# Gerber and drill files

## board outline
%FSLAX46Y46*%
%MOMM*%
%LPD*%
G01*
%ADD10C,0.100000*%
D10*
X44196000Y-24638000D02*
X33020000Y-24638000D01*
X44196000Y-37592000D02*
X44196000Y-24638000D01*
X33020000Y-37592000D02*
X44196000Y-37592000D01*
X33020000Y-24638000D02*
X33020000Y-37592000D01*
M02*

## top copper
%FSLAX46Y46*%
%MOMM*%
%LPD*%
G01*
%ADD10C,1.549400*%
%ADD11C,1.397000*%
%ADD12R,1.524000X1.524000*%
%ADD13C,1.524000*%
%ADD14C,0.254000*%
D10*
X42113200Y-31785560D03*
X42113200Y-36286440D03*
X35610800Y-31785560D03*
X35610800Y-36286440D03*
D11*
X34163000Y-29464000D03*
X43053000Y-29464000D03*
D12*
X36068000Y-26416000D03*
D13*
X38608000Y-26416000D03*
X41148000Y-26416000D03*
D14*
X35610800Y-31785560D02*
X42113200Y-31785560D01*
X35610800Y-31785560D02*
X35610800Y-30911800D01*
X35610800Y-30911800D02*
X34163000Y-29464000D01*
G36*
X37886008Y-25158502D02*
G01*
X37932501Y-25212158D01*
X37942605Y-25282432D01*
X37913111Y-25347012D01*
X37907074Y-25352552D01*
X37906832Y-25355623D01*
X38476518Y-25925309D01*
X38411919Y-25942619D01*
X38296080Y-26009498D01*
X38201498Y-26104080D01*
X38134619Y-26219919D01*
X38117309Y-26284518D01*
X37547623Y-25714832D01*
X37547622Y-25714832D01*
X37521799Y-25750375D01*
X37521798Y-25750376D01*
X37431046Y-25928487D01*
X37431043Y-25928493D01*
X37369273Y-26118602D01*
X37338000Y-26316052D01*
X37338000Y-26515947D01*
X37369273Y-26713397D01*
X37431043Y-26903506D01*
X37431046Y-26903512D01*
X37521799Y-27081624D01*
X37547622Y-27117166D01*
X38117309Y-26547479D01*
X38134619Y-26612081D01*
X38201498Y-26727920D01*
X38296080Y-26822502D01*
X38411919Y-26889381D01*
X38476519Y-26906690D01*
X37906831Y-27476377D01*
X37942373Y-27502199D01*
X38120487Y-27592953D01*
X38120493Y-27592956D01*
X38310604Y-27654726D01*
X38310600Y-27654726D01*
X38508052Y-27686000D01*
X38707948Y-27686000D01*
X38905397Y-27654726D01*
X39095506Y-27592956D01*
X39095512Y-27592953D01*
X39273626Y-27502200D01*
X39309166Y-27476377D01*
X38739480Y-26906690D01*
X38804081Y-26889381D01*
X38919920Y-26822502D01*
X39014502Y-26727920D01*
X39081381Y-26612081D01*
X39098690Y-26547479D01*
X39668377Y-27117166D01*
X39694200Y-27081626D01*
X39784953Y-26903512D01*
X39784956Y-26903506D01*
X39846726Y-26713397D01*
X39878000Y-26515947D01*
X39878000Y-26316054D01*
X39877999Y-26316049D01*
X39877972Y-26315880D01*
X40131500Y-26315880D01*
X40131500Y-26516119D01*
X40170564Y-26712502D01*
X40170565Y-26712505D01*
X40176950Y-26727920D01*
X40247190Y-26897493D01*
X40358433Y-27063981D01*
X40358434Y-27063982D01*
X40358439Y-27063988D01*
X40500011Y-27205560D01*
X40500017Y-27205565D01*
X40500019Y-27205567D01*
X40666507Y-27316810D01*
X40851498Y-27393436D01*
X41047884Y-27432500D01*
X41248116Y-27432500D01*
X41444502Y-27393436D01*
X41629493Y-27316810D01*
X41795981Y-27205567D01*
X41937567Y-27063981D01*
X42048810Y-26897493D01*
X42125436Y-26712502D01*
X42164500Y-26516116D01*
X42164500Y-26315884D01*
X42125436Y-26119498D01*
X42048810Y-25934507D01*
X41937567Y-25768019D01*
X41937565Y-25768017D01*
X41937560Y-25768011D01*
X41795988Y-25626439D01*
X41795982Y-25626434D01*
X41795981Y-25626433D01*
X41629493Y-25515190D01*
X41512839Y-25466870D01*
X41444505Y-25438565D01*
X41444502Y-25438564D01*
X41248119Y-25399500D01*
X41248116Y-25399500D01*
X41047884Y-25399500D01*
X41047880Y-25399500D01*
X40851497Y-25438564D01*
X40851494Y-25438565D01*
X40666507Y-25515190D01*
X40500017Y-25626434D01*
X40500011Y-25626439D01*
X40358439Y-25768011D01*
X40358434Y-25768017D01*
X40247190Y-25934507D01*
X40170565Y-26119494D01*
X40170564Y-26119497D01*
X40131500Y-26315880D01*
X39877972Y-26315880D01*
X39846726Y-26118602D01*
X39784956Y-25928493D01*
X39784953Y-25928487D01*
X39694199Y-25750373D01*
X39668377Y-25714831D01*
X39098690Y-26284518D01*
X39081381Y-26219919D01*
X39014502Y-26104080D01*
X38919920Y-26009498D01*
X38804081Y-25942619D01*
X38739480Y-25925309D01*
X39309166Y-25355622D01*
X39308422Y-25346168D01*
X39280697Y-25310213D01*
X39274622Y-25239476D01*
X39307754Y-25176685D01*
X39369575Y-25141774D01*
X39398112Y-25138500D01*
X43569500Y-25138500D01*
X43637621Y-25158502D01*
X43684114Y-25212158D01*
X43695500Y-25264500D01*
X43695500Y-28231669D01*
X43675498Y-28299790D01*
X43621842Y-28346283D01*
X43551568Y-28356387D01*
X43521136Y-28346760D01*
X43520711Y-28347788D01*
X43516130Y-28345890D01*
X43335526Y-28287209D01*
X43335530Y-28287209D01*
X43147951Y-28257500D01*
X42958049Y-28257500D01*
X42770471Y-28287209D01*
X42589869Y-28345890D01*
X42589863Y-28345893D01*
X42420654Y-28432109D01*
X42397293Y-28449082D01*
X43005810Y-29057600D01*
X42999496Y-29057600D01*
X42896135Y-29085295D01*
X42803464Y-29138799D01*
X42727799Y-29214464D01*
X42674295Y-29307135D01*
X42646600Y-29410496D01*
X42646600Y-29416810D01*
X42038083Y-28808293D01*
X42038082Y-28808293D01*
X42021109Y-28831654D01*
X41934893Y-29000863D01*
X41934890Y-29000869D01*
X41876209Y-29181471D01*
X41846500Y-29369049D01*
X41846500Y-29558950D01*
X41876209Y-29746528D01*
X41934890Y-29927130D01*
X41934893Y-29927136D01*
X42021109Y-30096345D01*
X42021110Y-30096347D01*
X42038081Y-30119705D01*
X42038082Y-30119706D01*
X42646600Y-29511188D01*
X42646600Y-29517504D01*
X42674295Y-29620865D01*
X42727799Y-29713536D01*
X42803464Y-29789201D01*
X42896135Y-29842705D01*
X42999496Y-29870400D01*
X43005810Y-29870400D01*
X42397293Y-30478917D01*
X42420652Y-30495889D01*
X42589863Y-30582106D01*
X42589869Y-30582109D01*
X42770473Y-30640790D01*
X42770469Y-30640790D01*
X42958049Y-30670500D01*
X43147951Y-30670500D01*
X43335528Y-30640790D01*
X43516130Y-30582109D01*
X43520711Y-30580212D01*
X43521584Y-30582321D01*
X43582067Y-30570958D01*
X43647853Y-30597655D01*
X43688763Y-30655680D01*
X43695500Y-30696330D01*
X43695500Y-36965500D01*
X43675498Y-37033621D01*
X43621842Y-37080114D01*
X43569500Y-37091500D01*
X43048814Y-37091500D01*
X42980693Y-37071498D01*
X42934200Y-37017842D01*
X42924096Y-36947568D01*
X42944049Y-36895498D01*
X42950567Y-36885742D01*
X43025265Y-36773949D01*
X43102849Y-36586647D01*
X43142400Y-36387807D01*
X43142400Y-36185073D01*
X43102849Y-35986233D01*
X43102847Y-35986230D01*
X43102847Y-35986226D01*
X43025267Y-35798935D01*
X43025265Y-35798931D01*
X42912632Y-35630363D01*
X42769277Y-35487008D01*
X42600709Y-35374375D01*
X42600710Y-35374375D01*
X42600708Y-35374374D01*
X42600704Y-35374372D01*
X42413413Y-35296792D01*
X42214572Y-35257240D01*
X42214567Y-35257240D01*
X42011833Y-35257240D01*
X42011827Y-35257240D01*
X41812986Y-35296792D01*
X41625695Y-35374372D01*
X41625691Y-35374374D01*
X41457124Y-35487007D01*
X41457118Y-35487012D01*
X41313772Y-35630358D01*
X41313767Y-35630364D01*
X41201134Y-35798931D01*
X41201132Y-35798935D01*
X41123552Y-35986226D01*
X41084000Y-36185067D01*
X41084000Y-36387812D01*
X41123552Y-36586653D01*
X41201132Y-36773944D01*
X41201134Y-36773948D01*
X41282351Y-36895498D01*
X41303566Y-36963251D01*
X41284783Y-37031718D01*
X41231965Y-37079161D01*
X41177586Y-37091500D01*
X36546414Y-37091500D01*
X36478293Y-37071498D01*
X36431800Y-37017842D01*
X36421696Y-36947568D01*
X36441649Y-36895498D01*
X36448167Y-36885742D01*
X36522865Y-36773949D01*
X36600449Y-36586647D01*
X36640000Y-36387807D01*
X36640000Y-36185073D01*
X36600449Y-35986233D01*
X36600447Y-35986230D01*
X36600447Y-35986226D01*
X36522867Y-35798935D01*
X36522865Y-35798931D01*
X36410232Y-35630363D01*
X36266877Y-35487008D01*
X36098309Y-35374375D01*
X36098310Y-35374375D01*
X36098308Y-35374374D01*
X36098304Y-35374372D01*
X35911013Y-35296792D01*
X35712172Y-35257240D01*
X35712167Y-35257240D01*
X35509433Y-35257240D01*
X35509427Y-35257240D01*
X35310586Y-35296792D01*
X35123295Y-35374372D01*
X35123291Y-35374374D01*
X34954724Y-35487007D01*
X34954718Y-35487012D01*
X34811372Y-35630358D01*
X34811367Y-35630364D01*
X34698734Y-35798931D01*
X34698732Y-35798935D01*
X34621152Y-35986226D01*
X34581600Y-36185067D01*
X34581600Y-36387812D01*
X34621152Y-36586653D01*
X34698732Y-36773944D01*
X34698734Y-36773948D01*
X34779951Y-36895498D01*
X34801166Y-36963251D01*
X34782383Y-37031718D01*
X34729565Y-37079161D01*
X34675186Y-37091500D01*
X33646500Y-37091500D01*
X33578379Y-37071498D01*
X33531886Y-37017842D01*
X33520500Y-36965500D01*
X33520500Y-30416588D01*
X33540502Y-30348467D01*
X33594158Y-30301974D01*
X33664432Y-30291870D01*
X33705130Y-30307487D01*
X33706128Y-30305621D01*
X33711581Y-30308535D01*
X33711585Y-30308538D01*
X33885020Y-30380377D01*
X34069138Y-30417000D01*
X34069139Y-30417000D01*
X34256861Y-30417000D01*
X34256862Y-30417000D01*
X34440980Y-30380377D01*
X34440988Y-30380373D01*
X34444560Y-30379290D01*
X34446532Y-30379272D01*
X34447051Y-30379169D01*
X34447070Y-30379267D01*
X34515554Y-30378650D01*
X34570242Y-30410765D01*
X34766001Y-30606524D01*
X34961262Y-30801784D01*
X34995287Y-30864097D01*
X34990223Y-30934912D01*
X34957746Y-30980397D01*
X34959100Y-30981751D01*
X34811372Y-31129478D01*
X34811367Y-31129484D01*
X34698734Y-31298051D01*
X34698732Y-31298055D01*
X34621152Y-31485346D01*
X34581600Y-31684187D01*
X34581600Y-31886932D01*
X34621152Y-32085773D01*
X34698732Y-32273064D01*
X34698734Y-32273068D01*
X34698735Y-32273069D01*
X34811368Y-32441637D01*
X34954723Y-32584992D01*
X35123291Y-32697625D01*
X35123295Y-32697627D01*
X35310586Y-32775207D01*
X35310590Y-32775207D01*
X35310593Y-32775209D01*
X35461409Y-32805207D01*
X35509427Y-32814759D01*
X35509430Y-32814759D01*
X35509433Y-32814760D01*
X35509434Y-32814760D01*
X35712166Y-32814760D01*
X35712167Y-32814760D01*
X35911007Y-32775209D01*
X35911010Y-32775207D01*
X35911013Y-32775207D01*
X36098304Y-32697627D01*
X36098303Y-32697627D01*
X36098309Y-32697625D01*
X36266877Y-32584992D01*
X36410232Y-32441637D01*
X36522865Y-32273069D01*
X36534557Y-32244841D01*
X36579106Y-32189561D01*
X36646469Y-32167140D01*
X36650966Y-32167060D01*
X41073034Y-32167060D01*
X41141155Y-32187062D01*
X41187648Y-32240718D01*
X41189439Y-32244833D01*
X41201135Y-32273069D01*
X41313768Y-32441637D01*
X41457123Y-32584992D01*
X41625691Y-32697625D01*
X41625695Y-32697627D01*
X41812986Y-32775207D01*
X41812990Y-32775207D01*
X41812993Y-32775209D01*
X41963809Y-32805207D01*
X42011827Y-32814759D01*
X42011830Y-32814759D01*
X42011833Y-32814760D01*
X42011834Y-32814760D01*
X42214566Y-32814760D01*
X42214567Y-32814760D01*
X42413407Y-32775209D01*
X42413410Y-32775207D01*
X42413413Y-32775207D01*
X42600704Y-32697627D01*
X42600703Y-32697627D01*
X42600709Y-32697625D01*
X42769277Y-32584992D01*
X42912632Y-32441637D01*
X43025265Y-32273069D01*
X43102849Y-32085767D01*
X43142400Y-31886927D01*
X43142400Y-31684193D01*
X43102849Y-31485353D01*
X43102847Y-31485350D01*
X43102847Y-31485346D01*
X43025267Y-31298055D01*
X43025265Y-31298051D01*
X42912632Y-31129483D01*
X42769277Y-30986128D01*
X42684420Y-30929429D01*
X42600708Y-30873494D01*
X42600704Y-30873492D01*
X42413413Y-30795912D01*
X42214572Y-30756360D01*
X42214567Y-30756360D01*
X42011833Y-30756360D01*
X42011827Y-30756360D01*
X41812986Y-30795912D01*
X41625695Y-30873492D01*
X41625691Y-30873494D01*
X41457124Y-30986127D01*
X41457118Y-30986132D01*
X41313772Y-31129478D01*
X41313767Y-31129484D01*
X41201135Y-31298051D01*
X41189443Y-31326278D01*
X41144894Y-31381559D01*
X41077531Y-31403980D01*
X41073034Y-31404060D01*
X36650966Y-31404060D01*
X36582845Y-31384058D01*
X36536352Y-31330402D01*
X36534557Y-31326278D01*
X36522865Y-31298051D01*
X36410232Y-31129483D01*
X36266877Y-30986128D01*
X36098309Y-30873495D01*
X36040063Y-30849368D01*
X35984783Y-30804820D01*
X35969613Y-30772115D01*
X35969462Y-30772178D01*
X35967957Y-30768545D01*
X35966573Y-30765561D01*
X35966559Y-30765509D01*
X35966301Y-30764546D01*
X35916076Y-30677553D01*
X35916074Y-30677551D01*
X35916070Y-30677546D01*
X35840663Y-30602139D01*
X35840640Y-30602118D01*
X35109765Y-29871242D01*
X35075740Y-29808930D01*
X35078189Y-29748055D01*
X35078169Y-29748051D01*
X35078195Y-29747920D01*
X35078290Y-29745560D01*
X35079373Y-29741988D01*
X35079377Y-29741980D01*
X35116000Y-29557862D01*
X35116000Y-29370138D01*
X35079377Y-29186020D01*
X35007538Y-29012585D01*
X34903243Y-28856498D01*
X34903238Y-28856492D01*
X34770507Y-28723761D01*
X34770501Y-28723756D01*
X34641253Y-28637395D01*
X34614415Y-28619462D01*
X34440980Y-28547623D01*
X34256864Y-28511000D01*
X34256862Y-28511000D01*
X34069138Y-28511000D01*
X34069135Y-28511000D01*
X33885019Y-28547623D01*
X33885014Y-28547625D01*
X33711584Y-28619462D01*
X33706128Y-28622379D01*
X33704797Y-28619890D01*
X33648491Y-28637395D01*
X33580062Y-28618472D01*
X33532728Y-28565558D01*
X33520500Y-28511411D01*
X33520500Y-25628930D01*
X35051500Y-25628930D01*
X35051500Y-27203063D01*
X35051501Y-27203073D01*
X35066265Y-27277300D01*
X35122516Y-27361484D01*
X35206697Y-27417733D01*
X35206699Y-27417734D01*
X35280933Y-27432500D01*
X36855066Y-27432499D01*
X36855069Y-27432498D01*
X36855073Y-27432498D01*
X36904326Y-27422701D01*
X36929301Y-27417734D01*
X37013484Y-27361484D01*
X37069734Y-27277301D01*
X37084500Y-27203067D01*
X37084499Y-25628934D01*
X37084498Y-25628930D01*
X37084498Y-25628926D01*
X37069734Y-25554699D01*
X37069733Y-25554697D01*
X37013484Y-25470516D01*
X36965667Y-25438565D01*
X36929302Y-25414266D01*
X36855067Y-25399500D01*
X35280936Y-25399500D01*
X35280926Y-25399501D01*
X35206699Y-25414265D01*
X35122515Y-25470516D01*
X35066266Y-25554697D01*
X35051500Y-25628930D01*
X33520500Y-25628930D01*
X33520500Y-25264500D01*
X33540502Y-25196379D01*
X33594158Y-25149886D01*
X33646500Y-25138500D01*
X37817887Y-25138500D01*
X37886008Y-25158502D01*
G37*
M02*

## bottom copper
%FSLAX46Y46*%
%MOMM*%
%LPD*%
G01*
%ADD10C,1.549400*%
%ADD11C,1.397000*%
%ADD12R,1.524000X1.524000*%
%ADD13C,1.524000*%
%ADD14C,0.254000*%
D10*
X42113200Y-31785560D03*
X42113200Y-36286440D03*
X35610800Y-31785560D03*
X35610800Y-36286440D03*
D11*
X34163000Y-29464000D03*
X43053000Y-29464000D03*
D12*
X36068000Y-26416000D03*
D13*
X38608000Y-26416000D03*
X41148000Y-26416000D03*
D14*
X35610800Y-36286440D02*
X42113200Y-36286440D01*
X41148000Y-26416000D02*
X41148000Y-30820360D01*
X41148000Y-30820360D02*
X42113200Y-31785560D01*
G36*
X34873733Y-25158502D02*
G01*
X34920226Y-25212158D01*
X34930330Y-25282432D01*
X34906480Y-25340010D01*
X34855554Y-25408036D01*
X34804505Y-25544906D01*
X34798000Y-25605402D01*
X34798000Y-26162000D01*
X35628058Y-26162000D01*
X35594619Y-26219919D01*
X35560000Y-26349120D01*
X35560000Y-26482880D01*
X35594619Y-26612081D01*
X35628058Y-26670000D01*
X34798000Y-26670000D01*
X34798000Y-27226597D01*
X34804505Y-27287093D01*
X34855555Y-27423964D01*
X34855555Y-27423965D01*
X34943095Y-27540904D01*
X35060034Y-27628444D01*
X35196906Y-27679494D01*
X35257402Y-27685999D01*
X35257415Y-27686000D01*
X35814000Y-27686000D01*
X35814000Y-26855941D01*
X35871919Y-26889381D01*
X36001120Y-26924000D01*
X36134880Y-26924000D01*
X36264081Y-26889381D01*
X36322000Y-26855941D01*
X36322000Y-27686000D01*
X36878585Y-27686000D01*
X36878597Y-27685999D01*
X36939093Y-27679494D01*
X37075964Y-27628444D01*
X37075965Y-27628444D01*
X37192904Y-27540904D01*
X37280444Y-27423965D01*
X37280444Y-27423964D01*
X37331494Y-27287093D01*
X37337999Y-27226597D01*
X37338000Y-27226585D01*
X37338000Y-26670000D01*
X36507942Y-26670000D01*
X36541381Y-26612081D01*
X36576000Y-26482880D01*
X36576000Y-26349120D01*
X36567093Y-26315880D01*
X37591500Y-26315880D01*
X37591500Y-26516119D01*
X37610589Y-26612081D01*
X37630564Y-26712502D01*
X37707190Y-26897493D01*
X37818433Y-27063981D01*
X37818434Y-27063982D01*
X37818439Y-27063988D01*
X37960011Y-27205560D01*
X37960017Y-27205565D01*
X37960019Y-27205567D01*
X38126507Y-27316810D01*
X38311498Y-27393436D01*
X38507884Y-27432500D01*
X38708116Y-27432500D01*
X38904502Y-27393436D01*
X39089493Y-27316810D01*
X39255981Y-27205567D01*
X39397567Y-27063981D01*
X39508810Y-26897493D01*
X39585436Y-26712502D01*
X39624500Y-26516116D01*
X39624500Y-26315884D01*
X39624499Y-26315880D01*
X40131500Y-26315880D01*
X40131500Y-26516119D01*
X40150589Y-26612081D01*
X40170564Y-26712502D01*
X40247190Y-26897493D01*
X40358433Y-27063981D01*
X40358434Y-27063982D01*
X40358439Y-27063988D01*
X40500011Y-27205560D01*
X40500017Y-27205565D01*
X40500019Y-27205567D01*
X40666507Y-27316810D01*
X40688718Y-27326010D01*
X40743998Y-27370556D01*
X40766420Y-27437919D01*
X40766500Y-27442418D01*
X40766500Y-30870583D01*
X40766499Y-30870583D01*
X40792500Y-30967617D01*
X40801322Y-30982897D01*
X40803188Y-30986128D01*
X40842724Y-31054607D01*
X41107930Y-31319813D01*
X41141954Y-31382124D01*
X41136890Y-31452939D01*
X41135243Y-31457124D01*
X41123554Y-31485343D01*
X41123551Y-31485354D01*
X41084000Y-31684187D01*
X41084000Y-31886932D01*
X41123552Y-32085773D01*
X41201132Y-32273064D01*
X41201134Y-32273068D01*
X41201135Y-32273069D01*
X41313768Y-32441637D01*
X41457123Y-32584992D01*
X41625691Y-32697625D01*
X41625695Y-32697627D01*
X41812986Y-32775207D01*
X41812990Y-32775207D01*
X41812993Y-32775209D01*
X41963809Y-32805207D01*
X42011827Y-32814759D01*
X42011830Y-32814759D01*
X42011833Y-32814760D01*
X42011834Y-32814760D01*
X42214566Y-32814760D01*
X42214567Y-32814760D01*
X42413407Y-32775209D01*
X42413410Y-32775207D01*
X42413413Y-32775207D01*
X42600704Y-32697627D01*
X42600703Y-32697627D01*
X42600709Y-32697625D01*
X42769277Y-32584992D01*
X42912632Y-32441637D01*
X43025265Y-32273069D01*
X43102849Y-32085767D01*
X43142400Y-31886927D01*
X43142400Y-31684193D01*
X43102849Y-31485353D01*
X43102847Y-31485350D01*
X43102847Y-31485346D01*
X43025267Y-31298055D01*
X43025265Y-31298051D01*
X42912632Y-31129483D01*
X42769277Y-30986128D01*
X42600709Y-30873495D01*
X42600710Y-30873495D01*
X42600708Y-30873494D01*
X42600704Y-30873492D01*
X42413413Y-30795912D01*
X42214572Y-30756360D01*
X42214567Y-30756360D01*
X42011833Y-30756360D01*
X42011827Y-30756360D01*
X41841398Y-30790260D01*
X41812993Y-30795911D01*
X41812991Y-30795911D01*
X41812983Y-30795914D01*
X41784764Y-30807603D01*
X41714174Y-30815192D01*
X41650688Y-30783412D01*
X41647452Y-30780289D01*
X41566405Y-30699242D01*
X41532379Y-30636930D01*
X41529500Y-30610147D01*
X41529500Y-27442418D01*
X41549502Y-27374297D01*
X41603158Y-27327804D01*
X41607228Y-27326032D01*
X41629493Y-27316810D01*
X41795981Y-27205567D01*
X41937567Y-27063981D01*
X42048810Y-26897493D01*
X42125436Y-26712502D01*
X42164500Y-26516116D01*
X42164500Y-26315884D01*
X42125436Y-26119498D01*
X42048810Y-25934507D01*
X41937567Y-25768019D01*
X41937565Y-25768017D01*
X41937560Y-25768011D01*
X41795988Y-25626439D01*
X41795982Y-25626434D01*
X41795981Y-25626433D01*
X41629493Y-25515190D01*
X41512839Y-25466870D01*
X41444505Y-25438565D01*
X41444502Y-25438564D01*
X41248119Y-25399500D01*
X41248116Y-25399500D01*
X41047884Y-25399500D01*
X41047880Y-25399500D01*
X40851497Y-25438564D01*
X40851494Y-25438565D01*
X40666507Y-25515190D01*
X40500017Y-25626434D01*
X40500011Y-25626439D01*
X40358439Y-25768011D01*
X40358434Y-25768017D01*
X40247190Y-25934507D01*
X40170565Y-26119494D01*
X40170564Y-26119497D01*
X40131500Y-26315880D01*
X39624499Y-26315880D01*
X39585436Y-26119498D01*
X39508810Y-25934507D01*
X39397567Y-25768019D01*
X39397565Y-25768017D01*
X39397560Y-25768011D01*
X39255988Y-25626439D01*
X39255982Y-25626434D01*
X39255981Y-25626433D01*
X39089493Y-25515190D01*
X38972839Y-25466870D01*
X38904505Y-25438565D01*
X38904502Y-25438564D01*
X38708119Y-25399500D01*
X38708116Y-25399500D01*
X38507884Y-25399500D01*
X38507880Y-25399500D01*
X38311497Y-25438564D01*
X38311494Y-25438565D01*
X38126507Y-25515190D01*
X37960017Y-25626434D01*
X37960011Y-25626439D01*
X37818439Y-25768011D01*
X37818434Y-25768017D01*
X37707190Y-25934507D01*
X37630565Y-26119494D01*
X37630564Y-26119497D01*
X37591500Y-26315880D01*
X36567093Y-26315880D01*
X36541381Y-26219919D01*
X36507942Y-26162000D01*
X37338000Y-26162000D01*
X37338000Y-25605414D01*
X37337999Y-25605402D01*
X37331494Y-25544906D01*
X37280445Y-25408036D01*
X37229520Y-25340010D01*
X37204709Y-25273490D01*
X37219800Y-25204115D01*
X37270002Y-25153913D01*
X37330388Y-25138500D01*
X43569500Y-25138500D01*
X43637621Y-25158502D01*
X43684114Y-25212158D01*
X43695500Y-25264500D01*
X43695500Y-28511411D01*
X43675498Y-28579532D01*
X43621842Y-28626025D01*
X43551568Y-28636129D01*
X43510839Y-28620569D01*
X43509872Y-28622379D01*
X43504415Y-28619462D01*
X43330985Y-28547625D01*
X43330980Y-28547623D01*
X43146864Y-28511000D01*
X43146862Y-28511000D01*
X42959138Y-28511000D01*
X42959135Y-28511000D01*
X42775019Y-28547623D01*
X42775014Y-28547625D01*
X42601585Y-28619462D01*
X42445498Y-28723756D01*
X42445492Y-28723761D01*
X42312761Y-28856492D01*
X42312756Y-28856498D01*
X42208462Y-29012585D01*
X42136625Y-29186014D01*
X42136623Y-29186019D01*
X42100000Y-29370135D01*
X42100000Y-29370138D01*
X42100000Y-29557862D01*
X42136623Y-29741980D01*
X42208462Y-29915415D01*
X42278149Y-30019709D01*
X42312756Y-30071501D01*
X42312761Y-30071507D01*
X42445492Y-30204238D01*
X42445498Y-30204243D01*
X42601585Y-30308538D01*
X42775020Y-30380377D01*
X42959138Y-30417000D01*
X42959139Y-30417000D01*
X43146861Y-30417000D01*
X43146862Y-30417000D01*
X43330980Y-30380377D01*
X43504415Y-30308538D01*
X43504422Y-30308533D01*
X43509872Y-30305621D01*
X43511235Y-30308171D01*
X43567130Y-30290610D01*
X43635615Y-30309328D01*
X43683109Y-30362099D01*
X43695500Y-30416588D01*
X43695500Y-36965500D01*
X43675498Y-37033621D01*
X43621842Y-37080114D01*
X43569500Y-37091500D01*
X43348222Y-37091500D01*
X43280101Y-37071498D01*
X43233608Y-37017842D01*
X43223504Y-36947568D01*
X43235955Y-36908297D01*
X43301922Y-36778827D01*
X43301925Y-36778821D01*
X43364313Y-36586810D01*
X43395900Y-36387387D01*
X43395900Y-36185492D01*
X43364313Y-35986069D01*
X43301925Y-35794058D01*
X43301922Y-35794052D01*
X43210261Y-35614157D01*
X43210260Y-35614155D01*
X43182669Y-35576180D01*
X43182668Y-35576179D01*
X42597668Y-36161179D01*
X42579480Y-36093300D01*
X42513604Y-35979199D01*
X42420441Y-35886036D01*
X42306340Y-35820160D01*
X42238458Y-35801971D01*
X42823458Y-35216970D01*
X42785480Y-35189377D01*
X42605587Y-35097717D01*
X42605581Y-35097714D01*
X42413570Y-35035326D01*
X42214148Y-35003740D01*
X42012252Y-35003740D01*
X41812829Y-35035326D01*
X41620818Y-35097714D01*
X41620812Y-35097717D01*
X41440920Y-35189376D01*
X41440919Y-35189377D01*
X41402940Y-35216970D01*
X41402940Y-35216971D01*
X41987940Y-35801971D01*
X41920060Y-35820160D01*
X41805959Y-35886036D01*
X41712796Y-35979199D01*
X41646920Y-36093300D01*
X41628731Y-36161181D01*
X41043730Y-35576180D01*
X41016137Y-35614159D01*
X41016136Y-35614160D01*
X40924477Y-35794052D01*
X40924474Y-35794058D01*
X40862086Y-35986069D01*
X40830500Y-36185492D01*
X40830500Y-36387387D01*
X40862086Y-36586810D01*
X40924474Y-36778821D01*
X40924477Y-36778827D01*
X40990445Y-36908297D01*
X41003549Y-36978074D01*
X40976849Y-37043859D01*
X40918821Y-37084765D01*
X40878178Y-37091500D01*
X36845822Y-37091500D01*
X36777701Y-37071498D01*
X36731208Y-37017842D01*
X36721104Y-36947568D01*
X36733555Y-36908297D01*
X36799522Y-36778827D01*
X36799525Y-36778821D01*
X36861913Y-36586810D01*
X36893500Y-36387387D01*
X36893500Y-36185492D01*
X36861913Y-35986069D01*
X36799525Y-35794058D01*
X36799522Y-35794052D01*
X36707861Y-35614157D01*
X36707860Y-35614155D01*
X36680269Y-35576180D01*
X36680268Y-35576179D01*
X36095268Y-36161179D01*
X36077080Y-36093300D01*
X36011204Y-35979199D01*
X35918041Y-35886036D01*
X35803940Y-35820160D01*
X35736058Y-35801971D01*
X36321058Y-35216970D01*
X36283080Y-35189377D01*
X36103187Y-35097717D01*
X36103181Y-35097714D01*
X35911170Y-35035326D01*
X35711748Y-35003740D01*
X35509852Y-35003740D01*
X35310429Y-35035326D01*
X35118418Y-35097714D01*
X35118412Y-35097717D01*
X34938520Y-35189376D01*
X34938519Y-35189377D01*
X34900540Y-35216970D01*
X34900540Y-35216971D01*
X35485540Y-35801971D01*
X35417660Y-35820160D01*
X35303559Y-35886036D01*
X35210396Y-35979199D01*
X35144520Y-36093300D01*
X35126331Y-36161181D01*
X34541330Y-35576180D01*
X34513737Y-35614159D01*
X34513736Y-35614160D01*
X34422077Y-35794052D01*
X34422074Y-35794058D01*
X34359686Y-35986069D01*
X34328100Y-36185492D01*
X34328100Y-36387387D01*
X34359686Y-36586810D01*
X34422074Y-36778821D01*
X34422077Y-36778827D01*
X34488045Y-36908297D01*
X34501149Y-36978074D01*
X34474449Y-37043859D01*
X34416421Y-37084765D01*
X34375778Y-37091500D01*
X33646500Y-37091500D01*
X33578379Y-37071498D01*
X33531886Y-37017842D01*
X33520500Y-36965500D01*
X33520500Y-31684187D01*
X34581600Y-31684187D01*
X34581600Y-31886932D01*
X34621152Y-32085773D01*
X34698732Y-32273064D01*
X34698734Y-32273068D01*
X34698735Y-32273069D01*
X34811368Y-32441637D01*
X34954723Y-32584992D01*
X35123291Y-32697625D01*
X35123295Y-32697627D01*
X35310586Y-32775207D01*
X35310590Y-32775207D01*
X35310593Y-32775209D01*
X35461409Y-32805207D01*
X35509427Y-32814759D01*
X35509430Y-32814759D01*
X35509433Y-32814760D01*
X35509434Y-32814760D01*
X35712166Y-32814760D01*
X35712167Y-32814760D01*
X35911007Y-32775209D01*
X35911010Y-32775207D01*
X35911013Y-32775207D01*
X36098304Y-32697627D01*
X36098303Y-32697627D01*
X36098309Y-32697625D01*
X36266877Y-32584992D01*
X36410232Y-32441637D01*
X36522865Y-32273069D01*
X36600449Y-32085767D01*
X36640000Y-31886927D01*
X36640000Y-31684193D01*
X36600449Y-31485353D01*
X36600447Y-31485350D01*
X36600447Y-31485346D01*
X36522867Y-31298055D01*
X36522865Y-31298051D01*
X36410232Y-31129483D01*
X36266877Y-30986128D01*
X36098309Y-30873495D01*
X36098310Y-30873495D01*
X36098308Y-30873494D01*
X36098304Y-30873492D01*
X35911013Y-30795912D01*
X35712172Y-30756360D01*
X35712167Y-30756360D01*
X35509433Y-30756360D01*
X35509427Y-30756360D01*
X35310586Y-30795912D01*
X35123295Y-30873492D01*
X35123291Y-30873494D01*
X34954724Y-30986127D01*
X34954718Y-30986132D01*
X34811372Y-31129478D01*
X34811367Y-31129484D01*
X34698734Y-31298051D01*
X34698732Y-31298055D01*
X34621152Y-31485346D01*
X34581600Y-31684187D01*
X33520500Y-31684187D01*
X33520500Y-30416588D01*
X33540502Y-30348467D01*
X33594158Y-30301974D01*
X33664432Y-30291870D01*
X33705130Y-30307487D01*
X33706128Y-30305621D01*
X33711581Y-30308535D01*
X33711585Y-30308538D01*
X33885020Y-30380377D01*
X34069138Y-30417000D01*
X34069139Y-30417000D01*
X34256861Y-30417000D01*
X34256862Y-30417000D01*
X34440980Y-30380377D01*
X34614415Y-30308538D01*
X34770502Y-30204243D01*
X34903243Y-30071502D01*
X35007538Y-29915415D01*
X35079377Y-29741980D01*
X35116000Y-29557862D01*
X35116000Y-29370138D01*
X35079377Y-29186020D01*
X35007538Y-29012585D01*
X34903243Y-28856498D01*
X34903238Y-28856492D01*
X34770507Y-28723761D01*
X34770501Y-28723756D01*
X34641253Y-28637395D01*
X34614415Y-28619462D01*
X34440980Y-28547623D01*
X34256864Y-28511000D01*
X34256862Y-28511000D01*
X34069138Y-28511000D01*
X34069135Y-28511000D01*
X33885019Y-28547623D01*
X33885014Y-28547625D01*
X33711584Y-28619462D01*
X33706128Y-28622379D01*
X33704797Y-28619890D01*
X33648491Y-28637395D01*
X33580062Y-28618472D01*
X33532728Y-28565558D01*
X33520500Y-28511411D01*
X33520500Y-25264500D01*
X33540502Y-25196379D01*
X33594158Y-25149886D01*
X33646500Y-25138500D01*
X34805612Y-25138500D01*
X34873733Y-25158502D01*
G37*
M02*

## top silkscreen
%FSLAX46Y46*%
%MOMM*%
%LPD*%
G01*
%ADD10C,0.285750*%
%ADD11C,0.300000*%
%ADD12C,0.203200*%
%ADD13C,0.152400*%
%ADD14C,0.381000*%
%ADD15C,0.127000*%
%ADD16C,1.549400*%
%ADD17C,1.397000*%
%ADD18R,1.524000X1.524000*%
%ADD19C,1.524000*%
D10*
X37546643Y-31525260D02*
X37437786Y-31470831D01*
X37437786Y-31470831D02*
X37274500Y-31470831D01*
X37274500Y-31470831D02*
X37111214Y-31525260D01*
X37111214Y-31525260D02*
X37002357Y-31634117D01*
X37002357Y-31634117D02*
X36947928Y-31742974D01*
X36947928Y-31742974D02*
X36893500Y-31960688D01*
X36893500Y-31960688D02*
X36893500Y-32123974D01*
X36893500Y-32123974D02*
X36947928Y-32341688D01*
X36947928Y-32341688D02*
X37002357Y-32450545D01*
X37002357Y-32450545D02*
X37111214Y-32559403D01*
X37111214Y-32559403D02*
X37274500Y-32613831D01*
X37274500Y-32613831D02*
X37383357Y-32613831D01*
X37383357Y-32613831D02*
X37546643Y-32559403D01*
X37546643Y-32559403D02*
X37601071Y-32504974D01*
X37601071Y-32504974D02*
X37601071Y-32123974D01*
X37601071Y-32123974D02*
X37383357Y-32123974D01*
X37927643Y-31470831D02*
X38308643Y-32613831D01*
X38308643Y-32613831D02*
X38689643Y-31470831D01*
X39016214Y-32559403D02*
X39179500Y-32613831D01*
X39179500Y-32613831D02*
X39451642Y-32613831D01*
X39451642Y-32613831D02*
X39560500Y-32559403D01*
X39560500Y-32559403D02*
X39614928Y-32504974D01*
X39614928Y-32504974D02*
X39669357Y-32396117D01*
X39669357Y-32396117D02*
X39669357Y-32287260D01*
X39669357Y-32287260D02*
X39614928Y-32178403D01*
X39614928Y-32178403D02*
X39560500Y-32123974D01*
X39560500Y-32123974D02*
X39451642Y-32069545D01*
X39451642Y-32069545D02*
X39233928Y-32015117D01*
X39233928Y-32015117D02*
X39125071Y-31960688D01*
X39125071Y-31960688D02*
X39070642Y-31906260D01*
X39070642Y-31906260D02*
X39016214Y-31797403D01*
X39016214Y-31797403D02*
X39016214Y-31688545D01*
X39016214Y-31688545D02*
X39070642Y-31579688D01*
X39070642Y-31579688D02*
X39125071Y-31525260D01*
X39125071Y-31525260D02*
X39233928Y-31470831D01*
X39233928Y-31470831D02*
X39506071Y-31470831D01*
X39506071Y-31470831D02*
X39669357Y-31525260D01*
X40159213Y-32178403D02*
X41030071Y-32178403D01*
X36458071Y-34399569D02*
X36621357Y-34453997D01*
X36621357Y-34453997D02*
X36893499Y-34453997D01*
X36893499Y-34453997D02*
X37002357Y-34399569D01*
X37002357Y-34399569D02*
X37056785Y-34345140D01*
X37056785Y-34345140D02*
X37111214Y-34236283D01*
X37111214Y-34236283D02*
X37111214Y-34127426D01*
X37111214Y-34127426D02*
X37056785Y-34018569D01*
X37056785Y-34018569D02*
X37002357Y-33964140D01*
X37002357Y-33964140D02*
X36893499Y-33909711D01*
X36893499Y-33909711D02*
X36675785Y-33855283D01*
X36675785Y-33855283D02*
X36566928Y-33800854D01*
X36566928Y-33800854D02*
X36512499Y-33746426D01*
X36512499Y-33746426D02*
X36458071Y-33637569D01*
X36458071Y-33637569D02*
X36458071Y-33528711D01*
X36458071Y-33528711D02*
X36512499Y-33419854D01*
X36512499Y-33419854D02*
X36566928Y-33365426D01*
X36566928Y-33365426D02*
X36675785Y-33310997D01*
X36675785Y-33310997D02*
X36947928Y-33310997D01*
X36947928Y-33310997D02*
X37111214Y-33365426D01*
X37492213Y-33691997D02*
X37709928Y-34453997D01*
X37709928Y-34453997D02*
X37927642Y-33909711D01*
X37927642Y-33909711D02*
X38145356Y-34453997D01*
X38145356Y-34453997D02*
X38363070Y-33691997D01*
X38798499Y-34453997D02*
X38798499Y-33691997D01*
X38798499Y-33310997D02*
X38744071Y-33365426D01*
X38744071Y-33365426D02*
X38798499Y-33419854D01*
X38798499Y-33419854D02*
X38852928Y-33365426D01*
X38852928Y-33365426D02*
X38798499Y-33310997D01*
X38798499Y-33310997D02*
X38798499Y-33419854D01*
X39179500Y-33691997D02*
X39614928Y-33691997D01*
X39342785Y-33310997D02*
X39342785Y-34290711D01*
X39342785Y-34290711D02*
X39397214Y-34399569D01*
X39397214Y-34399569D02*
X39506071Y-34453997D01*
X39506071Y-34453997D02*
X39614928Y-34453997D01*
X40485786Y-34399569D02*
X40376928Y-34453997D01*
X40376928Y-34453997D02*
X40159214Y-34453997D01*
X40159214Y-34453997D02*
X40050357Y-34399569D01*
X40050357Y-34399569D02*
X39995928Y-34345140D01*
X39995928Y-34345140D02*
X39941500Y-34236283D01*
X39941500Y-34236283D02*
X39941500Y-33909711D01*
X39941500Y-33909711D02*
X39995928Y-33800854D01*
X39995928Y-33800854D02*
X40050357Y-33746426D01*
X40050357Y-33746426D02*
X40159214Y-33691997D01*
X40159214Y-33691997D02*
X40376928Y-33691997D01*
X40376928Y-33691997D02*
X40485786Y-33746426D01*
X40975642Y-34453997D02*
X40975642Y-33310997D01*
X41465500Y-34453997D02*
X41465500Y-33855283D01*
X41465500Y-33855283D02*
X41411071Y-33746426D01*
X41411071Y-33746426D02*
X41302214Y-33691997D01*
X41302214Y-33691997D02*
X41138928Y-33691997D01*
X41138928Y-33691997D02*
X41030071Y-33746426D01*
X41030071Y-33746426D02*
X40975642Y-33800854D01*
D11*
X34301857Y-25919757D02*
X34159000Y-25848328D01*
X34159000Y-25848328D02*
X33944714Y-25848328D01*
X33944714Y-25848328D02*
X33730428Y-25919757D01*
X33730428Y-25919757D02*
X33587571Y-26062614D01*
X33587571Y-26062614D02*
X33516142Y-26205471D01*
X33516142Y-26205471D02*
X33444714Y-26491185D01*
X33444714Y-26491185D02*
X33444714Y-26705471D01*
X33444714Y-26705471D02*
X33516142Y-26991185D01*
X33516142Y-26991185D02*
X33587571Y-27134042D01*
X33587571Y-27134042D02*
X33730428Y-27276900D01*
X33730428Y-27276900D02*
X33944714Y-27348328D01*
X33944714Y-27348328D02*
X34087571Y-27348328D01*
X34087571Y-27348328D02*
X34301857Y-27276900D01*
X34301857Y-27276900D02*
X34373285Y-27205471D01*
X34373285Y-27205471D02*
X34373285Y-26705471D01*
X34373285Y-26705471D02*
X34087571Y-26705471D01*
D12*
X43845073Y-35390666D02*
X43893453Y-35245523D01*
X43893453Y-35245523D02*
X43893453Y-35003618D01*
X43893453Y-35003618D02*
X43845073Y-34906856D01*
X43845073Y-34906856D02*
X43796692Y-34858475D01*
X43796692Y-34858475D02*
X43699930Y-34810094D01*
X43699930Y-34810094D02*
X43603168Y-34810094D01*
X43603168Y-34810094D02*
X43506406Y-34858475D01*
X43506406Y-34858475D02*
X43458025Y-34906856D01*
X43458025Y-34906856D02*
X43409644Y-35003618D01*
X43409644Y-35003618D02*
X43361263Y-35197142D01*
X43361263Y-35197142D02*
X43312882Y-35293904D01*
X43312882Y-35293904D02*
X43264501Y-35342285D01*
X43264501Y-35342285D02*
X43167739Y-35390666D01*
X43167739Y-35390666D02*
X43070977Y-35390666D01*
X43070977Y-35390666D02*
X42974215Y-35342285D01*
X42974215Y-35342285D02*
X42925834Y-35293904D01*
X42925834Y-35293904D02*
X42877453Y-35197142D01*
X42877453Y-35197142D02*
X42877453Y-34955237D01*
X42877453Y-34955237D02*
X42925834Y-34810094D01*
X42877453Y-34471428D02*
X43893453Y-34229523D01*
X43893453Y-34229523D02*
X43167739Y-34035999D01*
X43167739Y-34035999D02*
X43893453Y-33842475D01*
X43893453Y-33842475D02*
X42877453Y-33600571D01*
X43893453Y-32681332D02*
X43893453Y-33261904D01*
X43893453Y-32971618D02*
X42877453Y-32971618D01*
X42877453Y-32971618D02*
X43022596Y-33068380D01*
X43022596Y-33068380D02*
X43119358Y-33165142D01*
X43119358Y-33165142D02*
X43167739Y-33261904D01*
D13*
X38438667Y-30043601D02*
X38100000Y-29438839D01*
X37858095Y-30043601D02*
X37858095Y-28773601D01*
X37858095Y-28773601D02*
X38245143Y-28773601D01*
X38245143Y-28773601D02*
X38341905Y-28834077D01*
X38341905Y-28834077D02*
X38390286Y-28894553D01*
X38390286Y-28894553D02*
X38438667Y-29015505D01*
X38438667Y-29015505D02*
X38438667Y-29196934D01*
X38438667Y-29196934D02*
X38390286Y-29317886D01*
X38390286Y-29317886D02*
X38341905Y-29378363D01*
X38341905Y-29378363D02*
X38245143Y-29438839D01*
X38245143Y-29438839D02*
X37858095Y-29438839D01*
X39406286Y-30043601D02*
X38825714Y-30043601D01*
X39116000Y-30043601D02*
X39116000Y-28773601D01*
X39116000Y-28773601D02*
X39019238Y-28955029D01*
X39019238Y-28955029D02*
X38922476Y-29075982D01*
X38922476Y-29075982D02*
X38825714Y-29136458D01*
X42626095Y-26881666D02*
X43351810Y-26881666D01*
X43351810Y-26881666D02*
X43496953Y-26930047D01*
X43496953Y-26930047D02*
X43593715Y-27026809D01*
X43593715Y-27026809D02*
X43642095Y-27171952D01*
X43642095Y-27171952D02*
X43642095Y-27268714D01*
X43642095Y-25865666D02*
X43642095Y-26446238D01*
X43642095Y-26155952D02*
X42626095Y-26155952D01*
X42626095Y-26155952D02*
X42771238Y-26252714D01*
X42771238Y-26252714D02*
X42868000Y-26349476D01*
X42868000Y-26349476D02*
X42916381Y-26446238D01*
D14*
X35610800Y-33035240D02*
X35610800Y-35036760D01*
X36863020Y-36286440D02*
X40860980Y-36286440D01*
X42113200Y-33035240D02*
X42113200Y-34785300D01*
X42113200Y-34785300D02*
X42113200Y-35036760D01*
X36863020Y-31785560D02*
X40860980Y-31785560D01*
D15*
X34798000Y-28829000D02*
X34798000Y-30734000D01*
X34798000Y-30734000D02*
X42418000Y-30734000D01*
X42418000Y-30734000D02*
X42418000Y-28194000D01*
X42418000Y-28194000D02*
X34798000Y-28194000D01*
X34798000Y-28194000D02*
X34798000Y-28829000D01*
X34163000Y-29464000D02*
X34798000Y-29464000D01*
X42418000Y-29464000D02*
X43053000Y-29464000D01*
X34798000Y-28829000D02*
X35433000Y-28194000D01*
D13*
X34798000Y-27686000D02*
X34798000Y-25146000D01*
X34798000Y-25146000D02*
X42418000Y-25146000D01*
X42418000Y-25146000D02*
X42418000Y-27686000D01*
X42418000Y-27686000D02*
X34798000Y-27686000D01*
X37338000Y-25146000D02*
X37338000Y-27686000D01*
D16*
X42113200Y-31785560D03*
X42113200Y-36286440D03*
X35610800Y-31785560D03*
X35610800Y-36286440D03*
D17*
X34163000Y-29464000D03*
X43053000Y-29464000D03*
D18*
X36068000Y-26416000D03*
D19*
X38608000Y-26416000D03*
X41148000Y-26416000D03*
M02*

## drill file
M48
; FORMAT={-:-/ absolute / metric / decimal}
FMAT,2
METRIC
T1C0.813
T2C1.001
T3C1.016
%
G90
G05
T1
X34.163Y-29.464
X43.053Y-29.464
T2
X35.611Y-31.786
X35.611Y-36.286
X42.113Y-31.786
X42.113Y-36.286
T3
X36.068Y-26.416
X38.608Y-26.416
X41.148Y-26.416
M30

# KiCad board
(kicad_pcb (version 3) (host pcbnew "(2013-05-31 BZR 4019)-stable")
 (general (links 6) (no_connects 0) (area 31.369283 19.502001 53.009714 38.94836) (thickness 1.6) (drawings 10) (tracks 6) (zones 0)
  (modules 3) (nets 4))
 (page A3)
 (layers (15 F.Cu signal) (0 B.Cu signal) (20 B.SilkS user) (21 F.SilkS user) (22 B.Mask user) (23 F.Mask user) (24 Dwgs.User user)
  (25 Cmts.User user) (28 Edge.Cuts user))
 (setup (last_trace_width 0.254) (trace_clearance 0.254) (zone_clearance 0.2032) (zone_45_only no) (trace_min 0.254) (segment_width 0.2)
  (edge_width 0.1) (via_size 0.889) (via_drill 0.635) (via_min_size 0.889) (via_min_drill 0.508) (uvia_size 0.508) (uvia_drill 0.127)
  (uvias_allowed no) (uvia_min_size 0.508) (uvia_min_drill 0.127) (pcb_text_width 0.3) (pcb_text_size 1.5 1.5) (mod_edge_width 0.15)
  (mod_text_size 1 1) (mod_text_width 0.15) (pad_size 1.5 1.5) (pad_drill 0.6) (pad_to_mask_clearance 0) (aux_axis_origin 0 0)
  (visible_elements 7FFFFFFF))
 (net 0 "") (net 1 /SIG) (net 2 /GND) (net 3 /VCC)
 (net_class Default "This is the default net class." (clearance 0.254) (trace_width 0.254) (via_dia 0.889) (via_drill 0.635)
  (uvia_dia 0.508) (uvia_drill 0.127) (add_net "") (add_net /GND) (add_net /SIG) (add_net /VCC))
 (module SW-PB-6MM (layer F.Cu) (at 38.862 34.036)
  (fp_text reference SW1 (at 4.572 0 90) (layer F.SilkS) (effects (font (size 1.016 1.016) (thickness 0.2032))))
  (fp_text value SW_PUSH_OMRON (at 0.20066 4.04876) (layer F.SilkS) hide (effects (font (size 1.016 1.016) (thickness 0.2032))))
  (fp_line (start -3.2512 -1.00076) (end -3.2512 1.00076) (layer F.SilkS) (width 0.381))
  (fp_line (start -1.99898 2.25044) (end 1.99898 2.25044) (layer F.SilkS) (width 0.381))
  (fp_line (start 3.2512 -1.00076) (end 3.2512 0.7493) (layer F.SilkS) (width 0.381))
  (fp_line (start 3.2512 0.7493) (end 3.2512 1.00076) (layer F.SilkS) (width 0.381))
  (fp_line (start -1.99898 -2.25044) (end 1.99898 -2.25044) (layer F.SilkS) (width 0.381))
  (pad 2 thru_hole circle (at 3.2512 -2.25044) (size 1.5494 1.5494) (drill 1.00076) (layers *.Cu *.Mask F.SilkS) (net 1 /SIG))
  (pad 4 thru_hole circle (at 3.2512 2.25044) (size 1.5494 1.5494) (drill 1.00076) (layers *.Cu *.Mask F.SilkS) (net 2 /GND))
  (pad 1 thru_hole circle (at -3.2512 -2.25044) (size 1.5494 1.5494) (drill 1.00076) (layers *.Cu *.Mask F.SilkS) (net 1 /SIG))
  (pad 3 thru_hole circle (at -3.2512 2.25044) (size 1.5494 1.5494) (drill 1.00076) (layers *.Cu *.Mask F.SilkS) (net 2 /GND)))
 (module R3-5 (layer F.Cu) (at 38.608 29.464)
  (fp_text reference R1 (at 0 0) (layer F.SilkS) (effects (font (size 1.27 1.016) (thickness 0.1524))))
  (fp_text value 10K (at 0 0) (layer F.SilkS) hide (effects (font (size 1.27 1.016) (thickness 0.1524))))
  (fp_line (start -3.81 -0.635) (end -3.81 1.27) (layer F.SilkS) (width 0.127))
  (fp_line (start -3.81 1.27) (end 3.81 1.27) (layer F.SilkS) (width 0.127))
  (fp_line (start 3.81 1.27) (end 3.81 -1.27) (layer F.SilkS) (width 0.127))
  (fp_line (start 3.81 -1.27) (end -3.81 -1.27) (layer F.SilkS) (width 0.127))
  (fp_line (start -3.81 -1.27) (end -3.81 -0.635) (layer F.SilkS) (width 0.127))
  (fp_line (start -4.445 0) (end -3.81 0) (layer F.SilkS) (width 0.127))
  (fp_line (start 3.81 0) (end 4.445 0) (layer F.SilkS) (width 0.127))
  (fp_line (start -3.81 -0.635) (end -3.175 -1.27) (layer F.SilkS) (width 0.127))
  (pad 1 thru_hole circle (at -4.445 0) (size 1.397 1.397) (drill 0.8128) (layers *.Cu *.Mask F.SilkS) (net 1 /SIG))
  (pad 2 thru_hole circle (at 4.445 0) (size 1.397 1.397) (drill 0.8128) (layers *.Cu *.Mask F.SilkS) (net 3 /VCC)))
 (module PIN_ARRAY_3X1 (layer F.Cu) (at 38.608 26.416)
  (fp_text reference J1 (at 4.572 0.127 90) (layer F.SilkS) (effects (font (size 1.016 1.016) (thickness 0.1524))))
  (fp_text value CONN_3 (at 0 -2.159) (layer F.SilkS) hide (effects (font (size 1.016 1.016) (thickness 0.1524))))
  (fp_line (start -3.81 1.27) (end -3.81 -1.27) (layer F.SilkS) (width 0.1524))
  (fp_line (start -3.81 -1.27) (end 3.81 -1.27) (layer F.SilkS) (width 0.1524))
  (fp_line (start 3.81 -1.27) (end 3.81 1.27) (layer F.SilkS) (width 0.1524))
  (fp_line (start 3.81 1.27) (end -3.81 1.27) (layer F.SilkS) (width 0.1524))
  (fp_line (start -1.27 -1.27) (end -1.27 1.27) (layer F.SilkS) (width 0.1524))
  (pad 1 thru_hole rect (at -2.54 0) (size 1.524 1.524) (drill 1.016) (layers *.Cu *.Mask F.SilkS) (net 2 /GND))
  (pad 2 thru_hole circle (at 0 0) (size 1.524 1.524) (drill 1.016) (layers *.Cu *.Mask F.SilkS) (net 3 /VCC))
  (pad 3 thru_hole circle (at 2.54 0) (size 1.524 1.524) (drill 1.016) (layers *.Cu *.Mask F.SilkS) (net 1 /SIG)))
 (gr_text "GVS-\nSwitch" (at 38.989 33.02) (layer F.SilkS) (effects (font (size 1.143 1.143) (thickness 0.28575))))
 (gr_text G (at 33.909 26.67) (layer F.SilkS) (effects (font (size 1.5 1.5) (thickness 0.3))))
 (gr_line (start 44.196 24.638) (end 33.02 24.638) (angle 90) (layer Edge.Cuts) (width 0.1))
 (gr_line (start 44.196 37.592) (end 44.196 24.638) (angle 90) (layer Edge.Cuts) (width 0.1))
 (gr_line (start 33.02 37.592) (end 44.196 37.592) (angle 90) (layer Edge.Cuts) (width 0.1))
 (gr_line (start 33.02 24.638) (end 33.02 37.592) (angle 90) (layer Edge.Cuts) (width 0.1))
 (segment (start 35.6108 36.28644) (end 42.1132 36.28644) (width 0.254) (layer B.Cu) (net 2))
 (segment (start 41.148 26.416) (end 41.148 30.82036) (width 0.254) (layer B.Cu) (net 1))
 (segment (start 41.148 30.82036) (end 42.1132 31.78556) (width 0.254) (layer B.Cu) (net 1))
 (segment (start 35.6108 31.78556) (end 42.1132 31.78556) (width 0.254) (layer F.Cu) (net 1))
 (segment (start 35.6108 31.78556) (end 35.6108 30.9118) (width 0.254) (layer F.Cu) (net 1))
 (segment (start 35.6108 30.9118) (end 34.163 29.464) (width 0.254) (layer F.Cu) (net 1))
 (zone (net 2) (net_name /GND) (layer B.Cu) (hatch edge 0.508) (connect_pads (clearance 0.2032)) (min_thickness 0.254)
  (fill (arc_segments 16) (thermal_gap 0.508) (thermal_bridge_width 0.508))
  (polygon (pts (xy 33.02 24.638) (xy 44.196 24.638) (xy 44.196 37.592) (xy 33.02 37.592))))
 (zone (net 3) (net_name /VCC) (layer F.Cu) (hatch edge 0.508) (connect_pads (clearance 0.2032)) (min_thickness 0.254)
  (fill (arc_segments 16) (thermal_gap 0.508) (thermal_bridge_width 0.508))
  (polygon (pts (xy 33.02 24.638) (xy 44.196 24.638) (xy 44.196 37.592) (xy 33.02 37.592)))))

